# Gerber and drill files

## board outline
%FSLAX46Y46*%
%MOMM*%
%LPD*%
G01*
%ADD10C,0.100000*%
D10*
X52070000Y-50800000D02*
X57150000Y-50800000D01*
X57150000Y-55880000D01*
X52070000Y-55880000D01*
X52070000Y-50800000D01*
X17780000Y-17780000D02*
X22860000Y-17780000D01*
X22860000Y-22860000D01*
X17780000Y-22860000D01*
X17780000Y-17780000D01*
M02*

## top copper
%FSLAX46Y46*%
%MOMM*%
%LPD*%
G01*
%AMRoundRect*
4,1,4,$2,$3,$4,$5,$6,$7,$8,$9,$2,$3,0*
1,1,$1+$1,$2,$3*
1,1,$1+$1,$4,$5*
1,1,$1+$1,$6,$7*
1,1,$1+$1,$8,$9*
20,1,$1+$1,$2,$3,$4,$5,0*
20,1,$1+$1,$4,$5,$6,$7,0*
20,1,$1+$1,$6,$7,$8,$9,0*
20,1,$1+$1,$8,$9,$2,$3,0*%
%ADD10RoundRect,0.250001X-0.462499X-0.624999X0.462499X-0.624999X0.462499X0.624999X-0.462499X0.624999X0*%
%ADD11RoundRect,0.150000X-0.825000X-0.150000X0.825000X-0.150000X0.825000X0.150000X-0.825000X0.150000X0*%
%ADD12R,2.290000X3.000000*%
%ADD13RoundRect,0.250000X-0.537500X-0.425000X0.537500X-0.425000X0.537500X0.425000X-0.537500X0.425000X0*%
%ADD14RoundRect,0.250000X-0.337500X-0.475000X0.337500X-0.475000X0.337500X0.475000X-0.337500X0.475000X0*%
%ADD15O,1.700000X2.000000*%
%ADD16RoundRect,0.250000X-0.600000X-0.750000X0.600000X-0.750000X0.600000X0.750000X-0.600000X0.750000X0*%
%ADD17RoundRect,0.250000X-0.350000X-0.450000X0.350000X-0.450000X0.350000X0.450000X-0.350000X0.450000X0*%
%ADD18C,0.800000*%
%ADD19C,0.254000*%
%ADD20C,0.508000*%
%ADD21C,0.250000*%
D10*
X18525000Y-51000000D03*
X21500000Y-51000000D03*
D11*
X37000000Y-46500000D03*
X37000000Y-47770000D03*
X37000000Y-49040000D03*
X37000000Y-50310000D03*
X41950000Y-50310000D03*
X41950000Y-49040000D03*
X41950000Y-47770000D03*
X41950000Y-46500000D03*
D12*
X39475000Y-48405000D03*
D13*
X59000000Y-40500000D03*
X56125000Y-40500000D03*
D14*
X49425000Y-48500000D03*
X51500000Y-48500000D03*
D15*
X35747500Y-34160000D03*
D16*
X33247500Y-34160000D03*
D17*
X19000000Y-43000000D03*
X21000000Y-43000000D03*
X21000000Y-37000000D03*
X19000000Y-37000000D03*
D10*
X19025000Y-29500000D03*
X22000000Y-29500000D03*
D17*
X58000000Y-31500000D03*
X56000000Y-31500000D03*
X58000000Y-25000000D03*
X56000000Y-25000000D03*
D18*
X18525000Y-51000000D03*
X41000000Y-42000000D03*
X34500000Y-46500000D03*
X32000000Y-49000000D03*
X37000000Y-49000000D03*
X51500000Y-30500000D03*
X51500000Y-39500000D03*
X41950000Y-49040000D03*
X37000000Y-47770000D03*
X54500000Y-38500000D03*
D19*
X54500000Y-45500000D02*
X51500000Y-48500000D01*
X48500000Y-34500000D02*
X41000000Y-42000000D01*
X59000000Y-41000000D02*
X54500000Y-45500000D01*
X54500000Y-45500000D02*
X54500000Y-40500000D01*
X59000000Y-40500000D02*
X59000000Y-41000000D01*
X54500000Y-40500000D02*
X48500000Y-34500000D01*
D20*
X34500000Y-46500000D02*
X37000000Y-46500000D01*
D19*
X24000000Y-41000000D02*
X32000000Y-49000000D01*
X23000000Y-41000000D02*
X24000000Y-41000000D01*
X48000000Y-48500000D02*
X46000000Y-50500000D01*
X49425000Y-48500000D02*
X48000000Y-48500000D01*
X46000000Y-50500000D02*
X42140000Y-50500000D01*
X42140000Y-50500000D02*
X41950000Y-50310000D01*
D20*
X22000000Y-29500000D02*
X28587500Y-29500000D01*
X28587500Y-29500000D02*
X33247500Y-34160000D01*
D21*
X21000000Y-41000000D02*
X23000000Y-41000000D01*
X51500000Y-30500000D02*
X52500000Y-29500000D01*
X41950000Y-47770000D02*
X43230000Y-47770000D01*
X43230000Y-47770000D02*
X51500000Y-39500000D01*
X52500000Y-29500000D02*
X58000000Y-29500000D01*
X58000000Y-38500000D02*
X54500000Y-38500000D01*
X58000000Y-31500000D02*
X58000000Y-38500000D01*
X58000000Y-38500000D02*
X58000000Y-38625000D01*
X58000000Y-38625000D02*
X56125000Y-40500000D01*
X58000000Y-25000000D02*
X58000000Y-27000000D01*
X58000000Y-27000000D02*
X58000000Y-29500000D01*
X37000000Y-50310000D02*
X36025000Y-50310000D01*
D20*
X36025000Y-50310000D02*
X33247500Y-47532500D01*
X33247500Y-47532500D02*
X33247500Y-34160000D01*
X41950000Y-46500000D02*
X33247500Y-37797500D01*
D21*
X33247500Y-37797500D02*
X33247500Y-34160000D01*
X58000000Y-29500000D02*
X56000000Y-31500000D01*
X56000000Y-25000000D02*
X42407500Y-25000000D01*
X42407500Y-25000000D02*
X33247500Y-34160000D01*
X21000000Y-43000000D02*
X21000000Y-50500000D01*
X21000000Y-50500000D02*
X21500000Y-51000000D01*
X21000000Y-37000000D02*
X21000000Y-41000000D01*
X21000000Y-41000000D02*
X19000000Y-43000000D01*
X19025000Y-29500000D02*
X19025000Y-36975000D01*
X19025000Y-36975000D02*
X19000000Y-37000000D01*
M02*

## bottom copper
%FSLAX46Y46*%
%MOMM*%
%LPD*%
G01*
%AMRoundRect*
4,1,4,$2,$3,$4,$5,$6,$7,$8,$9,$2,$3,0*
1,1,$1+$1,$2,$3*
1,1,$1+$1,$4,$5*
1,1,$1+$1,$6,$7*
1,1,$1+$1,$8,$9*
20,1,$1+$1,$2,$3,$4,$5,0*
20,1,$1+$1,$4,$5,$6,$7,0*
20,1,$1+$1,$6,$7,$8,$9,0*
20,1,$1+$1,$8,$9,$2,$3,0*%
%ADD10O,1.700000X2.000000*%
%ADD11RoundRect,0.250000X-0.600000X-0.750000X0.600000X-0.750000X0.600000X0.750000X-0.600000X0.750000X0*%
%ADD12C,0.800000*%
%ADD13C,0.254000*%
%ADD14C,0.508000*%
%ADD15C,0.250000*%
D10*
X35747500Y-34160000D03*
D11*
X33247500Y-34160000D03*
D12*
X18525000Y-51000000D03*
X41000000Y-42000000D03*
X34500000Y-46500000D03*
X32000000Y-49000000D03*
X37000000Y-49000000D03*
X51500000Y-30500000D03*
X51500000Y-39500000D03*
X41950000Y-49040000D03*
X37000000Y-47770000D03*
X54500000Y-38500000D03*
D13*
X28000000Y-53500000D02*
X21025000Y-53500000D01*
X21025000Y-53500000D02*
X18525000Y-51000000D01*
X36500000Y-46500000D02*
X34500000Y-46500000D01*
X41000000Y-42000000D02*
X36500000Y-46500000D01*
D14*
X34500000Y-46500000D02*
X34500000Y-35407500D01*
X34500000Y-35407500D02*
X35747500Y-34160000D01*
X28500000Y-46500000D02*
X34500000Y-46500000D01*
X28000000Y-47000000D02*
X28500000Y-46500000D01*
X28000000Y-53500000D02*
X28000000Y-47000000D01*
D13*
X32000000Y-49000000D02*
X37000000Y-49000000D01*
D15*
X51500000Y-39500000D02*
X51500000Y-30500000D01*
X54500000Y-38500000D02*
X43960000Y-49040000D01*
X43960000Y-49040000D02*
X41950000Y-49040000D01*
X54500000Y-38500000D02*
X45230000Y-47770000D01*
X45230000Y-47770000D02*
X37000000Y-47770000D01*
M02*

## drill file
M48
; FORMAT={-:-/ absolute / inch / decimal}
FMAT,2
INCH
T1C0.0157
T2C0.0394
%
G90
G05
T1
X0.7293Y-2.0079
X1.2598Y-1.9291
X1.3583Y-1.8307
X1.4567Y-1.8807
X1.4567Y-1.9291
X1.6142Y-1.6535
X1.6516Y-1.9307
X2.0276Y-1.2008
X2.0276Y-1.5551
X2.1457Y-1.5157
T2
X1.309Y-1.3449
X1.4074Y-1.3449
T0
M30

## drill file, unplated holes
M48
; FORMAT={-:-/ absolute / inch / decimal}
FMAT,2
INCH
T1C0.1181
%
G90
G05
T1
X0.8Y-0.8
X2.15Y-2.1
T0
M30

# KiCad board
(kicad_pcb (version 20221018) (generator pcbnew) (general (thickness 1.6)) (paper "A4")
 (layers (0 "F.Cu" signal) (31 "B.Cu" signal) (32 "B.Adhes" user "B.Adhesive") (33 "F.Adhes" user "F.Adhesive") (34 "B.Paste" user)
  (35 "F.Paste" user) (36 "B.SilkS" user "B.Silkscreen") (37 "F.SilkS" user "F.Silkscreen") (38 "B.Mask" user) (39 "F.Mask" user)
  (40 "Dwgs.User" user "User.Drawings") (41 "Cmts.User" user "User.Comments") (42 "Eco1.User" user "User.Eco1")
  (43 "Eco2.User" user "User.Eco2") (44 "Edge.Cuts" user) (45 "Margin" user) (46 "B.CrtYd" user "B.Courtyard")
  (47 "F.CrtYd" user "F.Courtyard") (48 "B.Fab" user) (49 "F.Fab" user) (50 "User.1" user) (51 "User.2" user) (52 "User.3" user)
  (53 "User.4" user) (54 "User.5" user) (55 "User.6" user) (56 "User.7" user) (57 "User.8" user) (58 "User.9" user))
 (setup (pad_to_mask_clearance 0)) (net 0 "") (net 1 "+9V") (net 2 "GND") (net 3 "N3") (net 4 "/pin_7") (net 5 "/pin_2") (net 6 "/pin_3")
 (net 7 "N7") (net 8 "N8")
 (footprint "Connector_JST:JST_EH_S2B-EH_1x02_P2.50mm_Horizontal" (layer "F.Cu") (at 33.2475 34.16)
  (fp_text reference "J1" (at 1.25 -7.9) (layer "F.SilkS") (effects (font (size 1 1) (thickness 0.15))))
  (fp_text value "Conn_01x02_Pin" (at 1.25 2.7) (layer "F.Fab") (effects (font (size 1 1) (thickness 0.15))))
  (pad "1" thru_hole roundrect (at 0 0) (size 1.7 2) (drill 1) (layers "*.Cu" "*.Mask") (roundrect_rratio 0.1470588235) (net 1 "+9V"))
  (pad "2" thru_hole oval (at 2.5 0) (size 1.7 2) (drill 1) (layers "*.Cu" "*.Mask") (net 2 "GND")))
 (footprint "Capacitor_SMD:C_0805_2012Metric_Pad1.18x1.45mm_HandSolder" (layer "F.Cu") (at 50.4625 48.5)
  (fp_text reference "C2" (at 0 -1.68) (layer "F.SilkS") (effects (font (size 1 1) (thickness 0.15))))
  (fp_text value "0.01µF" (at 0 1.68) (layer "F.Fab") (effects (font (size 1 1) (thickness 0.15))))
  (pad "1" smd roundrect (at -1.0375 0) (size 1.175 1.45) (layers "F.Cu" "F.Paste" "F.Mask") (roundrect_rratio 0.2127659574) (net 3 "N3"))
  (pad "2" smd roundrect (at 1.0375 0) (size 1.175 1.45) (layers "F.Cu" "F.Paste" "F.Mask") (roundrect_rratio 0.2127659574) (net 2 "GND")))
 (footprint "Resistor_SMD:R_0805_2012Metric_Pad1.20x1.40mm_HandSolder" (layer "F.Cu") (at 57 25)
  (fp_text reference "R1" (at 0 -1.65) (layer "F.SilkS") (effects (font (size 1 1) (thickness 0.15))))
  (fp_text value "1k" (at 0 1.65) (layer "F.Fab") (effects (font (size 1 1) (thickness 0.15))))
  (pad "1" smd roundrect (at -1 0) (size 1.2 1.4) (layers "F.Cu" "F.Paste" "F.Mask") (roundrect_rratio 0.2083333333) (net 1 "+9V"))
  (pad "2" smd roundrect (at 1 0) (size 1.2 1.4) (layers "F.Cu" "F.Paste" "F.Mask") (roundrect_rratio 0.2083333333) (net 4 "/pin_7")))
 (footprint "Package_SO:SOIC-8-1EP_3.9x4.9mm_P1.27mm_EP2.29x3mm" (layer "F.Cu") (at 39.475 48.405)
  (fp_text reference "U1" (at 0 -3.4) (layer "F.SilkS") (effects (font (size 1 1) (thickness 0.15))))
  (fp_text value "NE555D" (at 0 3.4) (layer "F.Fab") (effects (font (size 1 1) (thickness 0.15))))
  (pad "" smd roundrect (at -0.57 -0.75) (size 0.92 1.21) (layers "F.Paste") (roundrect_rratio 0.25))
  (pad "" smd roundrect (at -0.57 0.75) (size 0.92 1.21) (layers "F.Paste") (roundrect_rratio 0.25))
  (pad "" smd roundrect (at 0.57 -0.75) (size 0.92 1.21) (layers "F.Paste") (roundrect_rratio 0.25))
  (pad "" smd roundrect (at 0.57 0.75) (size 0.92 1.21) (layers "F.Paste") (roundrect_rratio 0.25))
  (pad "1" smd roundrect (at -2.475 -1.905) (size 1.95 0.6) (layers "F.Cu" "F.Paste" "F.Mask") (roundrect_rratio 0.25) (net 2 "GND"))
  (pad "2" smd roundrect (at -2.475 -0.635) (size 1.95 0.6) (layers "F.Cu" "F.Paste" "F.Mask") (roundrect_rratio 0.25) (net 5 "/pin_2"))
  (pad "3" smd roundrect (at -2.475 0.635) (size 1.95 0.6) (layers "F.Cu" "F.Paste" "F.Mask") (roundrect_rratio 0.25) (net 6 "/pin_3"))
  (pad "4" smd roundrect (at -2.475 1.905) (size 1.95 0.6) (layers "F.Cu" "F.Paste" "F.Mask") (roundrect_rratio 0.25) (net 1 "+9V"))
  (pad "5" smd roundrect (at 2.475 1.905) (size 1.95 0.6) (layers "F.Cu" "F.Paste" "F.Mask") (roundrect_rratio 0.25) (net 3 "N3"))
  (pad "6" smd roundrect (at 2.475 0.635) (size 1.95 0.6) (layers "F.Cu" "F.Paste" "F.Mask") (roundrect_rratio 0.25) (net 5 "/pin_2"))
  (pad "7" smd roundrect (at 2.475 -0.635) (size 1.95 0.6) (layers "F.Cu" "F.Paste" "F.Mask") (roundrect_rratio 0.25) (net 4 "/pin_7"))
  (pad "8" smd roundrect (at 2.475 -1.905) (size 1.95 0.6) (layers "F.Cu" "F.Paste" "F.Mask") (roundrect_rratio 0.25) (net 1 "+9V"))
  (pad "9" smd rect (at 0 0) (size 2.29 3) (layers "F.Cu" "F.Mask")))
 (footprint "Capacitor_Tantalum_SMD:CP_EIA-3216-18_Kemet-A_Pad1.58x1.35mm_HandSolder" (layer "F.Cu") (at 57.5625 40.5)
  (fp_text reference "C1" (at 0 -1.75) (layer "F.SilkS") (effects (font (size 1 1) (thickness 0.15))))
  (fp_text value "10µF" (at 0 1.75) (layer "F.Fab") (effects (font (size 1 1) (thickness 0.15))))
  (pad "1" smd roundrect (at -1.4375 0) (size 1.575 1.35) (layers "F.Cu" "F.Paste" "F.Mask") (roundrect_rratio 0.1851851852)
   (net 5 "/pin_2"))
  (pad "2" smd roundrect (at 1.4375 0) (size 1.575 1.35) (layers "F.Cu" "F.Paste" "F.Mask") (roundrect_rratio 0.1851851852) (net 2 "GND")))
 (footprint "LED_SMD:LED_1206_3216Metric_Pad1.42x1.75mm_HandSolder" (layer "F.Cu") (at 20.5125 29.5)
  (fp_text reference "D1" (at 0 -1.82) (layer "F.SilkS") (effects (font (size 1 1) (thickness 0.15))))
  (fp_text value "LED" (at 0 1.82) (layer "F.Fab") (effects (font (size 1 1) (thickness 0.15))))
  (pad "1" smd roundrect (at -1.4875 0) (size 1.425 1.75) (layers "F.Cu" "F.Paste" "F.Mask") (roundrect_rratio 0.1754392982) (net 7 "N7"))
  (pad "2" smd roundrect (at 1.4875 0) (size 1.425 1.75) (layers "F.Cu" "F.Paste" "F.Mask") (roundrect_rratio 0.1754392982) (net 1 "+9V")))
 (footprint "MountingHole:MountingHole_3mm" (layer "F.Cu") (at 54.61 53.34)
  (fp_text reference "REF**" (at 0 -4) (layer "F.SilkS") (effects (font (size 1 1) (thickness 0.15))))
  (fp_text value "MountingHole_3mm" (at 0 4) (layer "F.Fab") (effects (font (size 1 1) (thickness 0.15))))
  (pad "" np_thru_hole circle (at 0 0) (size 3 3) (drill 3) (layers "F&B.Cu" "*.Mask")))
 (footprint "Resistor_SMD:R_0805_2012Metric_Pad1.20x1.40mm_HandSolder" (layer "F.Cu") (at 20 43)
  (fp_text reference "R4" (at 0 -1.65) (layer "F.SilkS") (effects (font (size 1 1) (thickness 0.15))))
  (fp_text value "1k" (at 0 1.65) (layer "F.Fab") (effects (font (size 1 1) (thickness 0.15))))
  (pad "1" smd roundrect (at -1 0) (size 1.2 1.4) (layers "F.Cu" "F.Paste" "F.Mask") (roundrect_rratio 0.2083333333) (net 6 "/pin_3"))
  (pad "2" smd roundrect (at 1 0) (size 1.2 1.4) (layers "F.Cu" "F.Paste" "F.Mask") (roundrect_rratio 0.2083333333) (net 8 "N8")))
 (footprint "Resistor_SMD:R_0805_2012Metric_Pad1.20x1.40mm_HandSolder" (layer "F.Cu") (at 57 31.5)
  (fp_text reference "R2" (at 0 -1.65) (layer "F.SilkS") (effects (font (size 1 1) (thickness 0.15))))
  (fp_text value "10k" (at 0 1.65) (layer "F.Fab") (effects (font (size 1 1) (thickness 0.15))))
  (pad "1" smd roundrect (at -1 0) (size 1.2 1.4) (layers "F.Cu" "F.Paste" "F.Mask") (roundrect_rratio 0.2083333333) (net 4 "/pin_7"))
  (pad "2" smd roundrect (at 1 0) (size 1.2 1.4) (layers "F.Cu" "F.Paste" "F.Mask") (roundrect_rratio 0.2083333333) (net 5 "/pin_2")))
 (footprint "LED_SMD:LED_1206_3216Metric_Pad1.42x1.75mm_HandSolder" (layer "F.Cu") (at 20.0125 51)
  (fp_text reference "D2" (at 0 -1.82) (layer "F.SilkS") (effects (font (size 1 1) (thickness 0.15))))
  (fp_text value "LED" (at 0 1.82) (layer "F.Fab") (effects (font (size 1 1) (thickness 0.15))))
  (pad "1" smd roundrect (at -1.4875 0) (size 1.425 1.75) (layers "F.Cu" "F.Paste" "F.Mask") (roundrect_rratio 0.1754392982) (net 2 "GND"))
  (pad "2" smd roundrect (at 1.4875 0) (size 1.425 1.75) (layers "F.Cu" "F.Paste" "F.Mask") (roundrect_rratio 0.1754392982) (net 8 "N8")))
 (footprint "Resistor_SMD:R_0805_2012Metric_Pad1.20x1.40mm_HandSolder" (layer "F.Cu") (at 20 37)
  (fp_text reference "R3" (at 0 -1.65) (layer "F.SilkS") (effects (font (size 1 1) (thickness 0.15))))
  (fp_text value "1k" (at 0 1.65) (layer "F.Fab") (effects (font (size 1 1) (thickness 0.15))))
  (pad "1" smd roundrect (at -1 0) (size 1.2 1.4) (layers "F.Cu" "F.Paste" "F.Mask") (roundrect_rratio 0.2083333333) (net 7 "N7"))
  (pad "2" smd roundrect (at 1 0) (size 1.2 1.4) (layers "F.Cu" "F.Paste" "F.Mask") (roundrect_rratio 0.2083333333) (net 6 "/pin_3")))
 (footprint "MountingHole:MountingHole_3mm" (layer "F.Cu") (at 20.32 20.32)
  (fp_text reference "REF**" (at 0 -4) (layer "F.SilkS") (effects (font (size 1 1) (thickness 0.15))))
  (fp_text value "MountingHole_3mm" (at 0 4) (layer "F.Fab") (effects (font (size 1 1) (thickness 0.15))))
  (pad "" np_thru_hole circle (at 0 0) (size 3 3) (drill 3) (layers "*.Cu" "*.Mask")))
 (gr_rect (start 52.07 50.8) (end 57.15 55.88) (stroke (width 0.1) (type default)) (fill none) (layer "Edge.Cuts"))
 (gr_rect (start 17.78 17.78) (end 22.86 22.86) (stroke (width 0.1) (type default)) (fill none) (layer "Edge.Cuts"))
 (segment (start 58 38.5) (end 58 38.625) (width 0.25) (layer "F.Cu") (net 5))
 (segment (start 58 38.625) (end 56.125 40.5) (width 0.25) (layer "F.Cu") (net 5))
 (segment (start 58 38.5) (end 54.5 38.5) (width 0.25) (layer "F.Cu") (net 5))
 (segment (start 58 31.5) (end 58 38.5) (width 0.25) (layer "F.Cu") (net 5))
 (via (at 54.5 38.5) (size 0.8) (drill 0.4) (layers "F.Cu" "B.Cu") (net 5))
 (via (at 41.95 49.04) (size 0.8) (drill 0.4) (layers "F.Cu" "B.Cu") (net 5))
 (via (at 37 47.77) (size 0.8) (drill 0.4) (layers "F.Cu" "B.Cu") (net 5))
 (segment (start 43.96 49.04) (end 41.95 49.04) (width 0.25) (layer "B.Cu") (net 5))
 (segment (start 54.5 38.5) (end 43.96 49.04) (width 0.25) (layer "B.Cu") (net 5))
 (segment (start 54.5 38.5) (end 45.23 47.77) (width 0.25) (layer "B.Cu") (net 5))
 (segment (start 45.23 47.77) (end 37 47.77) (width 0.25) (layer "B.Cu") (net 5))
 (segment (start 59 41) (end 54.5 45.5) (width 0.254) (layer "F.Cu") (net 2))
 (segment (start 34.5 46.5) (end 37 46.5) (width 0.508) (layer "F.Cu") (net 2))
 (segment (start 54.5 45.5) (end 54.5 40.5) (width 0.254) (layer "F.Cu") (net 2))
 (segment (start 54.5 40.5) (end 48.5 34.5) (width 0.254) (layer "F.Cu") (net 2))
 (segment (start 59 40.5) (end 59 41) (width 0.254) (layer "F.Cu") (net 2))
 (segment (start 48.5 34.5) (end 41 42) (width 0.254) (layer "F.Cu") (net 2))
 (segment (start 54.5 45.5) (end 51.5 48.5) (width 0.254) (layer "F.Cu") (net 2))
 (via (at 41 42) (size 0.8) (drill 0.4) (layers "F.Cu" "B.Cu") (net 2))
 (via (at 18.525 51) (size 0.8) (drill 0.4) (layers "F.Cu" "B.Cu") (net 2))
 (via (at 34.5 46.5) (size 0.8) (drill 0.4) (layers "F.Cu" "B.Cu") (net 2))
 (segment (start 41 42) (end 36.5 46.5) (width 0.254) (layer "B.Cu") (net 2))
 (segment (start 34.5 46.5) (end 34.5 35.4075) (width 0.508) (layer "B.Cu") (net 2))
 (segment (start 28 53.5) (end 28 47) (width 0.508) (layer "B.Cu") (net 2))
 (segment (start 28.5 46.5) (end 34.5 46.5) (width 0.508) (layer "B.Cu") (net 2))
 (segment (start 34.5 35.4075) (end 35.7475 34.16) (width 0.508) (layer "B.Cu") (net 2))
 (segment (start 28 53.5) (end 21.025 53.5) (width 0.254) (layer "B.Cu") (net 2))
 (segment (start 28 47) (end 28.5 46.5) (width 0.508) (layer "B.Cu") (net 2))
 (segment (start 36.5 46.5) (end 34.5 46.5) (width 0.254) (layer "B.Cu") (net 2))
 (segment (start 21.025 53.5) (end 18.525 51) (width 0.254) (layer "B.Cu") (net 2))
 (segment (start 48 48.5) (end 46 50.5) (width 0.254) (layer "F.Cu") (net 3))
 (segment (start 42.14 50.5) (end 41.95 50.31) (width 0.254) (layer "F.Cu") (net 3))
 (segment (start 46 50.5) (end 42.14 50.5) (width 0.254) (layer "F.Cu") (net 3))
 (segment (start 49.425 48.5) (end 48 48.5) (width 0.254) (layer "F.Cu") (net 3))
 (segment (start 19.025 36.975) (end 19 37) (width 0.25) (layer "F.Cu") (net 7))
 (segment (start 19.025 29.5) (end 19.025 36.975) (width 0.25) (layer "F.Cu") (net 7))
 (segment (start 42.4075 25) (end 33.2475 34.16) (width 0.25) (layer "F.Cu") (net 1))
 (segment (start 33.2475 37.7975) (end 33.2475 34.16) (width 0.25) (layer "F.Cu") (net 1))
 (segment (start 28.5875 29.5) (end 33.2475 34.16) (width 0.508) (layer "F.Cu") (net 1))
 (segment (start 33.2475 47.5325) (end 33.2475 34.16) (width 0.508) (layer "F.Cu") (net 1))
 (segment (start 37 50.31) (end 36.025 50.31) (width 0.25) (layer "F.Cu") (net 1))
 (segment (start 22 29.5) (end 28.5875 29.5) (width 0.508) (layer "F.Cu") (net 1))
 (segment (start 41.95 46.5) (end 33.2475 37.7975) (width 0.508) (layer "F.Cu") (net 1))
 (segment (start 56 25) (end 42.4075 25) (width 0.25) (layer "F.Cu") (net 1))
 (segment (start 36.025 50.31) (end 33.2475 47.5325) (width 0.508) (layer "F.Cu") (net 1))
 (segment (start 21 50.5) (end 21.5 51) (width 0.25) (layer "F.Cu") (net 8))
 (segment (start 21 43) (end 21 50.5) (width 0.25) (layer "F.Cu") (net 8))
 (segment (start 51.5 30.5) (end 52.5 29.5) (width 0.25) (layer "F.Cu") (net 4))
 (segment (start 43.23 47.77) (end 51.5 39.5) (width 0.25) (layer "F.Cu") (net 4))
 (segment (start 58 25) (end 58 27) (width 0.25) (layer "F.Cu") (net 4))
 (segment (start 58 29.5) (end 56 31.5) (width 0.25) (layer "F.Cu") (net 4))
 (segment (start 41.95 47.77) (end 43.23 47.77) (width 0.25) (layer "F.Cu") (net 4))
 (segment (start 58 27) (end 58 29.5) (width 0.25) (layer "F.Cu") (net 4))
 (segment (start 52.5 29.5) (end 58 29.5) (width 0.25) (layer "F.Cu") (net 4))
 (via (at 51.5 30.5) (size 0.8) (drill 0.4) (layers "F.Cu" "B.Cu") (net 4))
 (via (at 51.5 39.5) (size 0.8) (drill 0.4) (layers "F.Cu" "B.Cu") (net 4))
 (segment (start 51.5 39.5) (end 51.5 30.5) (width 0.25) (layer "B.Cu") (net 4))
 (segment (start 21 37) (end 21 41) (width 0.25) (layer "F.Cu") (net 6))
 (segment (start 21 41) (end 19 43) (width 0.25) (layer "F.Cu") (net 6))
 (segment (start 24 41) (end 32 49) (width 0.254) (layer "F.Cu") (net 6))
 (segment (start 21 41) (end 23 41) (width 0.25) (layer "F.Cu") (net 6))
 (segment (start 23 41) (end 24 41) (width 0.254) (layer "F.Cu") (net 6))
 (via (at 32 49) (size 0.8) (drill 0.4) (layers "F.Cu" "B.Cu") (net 6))
 (via (at 37 49) (size 0.8) (drill 0.4) (layers "F.Cu" "B.Cu") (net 6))
 (segment (start 32 49) (end 37 49) (width 0.254) (layer "B.Cu") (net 6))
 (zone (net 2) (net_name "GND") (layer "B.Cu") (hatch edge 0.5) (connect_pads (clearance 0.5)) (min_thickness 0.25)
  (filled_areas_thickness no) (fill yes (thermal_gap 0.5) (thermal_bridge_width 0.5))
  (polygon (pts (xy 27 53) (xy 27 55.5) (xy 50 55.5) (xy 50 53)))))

